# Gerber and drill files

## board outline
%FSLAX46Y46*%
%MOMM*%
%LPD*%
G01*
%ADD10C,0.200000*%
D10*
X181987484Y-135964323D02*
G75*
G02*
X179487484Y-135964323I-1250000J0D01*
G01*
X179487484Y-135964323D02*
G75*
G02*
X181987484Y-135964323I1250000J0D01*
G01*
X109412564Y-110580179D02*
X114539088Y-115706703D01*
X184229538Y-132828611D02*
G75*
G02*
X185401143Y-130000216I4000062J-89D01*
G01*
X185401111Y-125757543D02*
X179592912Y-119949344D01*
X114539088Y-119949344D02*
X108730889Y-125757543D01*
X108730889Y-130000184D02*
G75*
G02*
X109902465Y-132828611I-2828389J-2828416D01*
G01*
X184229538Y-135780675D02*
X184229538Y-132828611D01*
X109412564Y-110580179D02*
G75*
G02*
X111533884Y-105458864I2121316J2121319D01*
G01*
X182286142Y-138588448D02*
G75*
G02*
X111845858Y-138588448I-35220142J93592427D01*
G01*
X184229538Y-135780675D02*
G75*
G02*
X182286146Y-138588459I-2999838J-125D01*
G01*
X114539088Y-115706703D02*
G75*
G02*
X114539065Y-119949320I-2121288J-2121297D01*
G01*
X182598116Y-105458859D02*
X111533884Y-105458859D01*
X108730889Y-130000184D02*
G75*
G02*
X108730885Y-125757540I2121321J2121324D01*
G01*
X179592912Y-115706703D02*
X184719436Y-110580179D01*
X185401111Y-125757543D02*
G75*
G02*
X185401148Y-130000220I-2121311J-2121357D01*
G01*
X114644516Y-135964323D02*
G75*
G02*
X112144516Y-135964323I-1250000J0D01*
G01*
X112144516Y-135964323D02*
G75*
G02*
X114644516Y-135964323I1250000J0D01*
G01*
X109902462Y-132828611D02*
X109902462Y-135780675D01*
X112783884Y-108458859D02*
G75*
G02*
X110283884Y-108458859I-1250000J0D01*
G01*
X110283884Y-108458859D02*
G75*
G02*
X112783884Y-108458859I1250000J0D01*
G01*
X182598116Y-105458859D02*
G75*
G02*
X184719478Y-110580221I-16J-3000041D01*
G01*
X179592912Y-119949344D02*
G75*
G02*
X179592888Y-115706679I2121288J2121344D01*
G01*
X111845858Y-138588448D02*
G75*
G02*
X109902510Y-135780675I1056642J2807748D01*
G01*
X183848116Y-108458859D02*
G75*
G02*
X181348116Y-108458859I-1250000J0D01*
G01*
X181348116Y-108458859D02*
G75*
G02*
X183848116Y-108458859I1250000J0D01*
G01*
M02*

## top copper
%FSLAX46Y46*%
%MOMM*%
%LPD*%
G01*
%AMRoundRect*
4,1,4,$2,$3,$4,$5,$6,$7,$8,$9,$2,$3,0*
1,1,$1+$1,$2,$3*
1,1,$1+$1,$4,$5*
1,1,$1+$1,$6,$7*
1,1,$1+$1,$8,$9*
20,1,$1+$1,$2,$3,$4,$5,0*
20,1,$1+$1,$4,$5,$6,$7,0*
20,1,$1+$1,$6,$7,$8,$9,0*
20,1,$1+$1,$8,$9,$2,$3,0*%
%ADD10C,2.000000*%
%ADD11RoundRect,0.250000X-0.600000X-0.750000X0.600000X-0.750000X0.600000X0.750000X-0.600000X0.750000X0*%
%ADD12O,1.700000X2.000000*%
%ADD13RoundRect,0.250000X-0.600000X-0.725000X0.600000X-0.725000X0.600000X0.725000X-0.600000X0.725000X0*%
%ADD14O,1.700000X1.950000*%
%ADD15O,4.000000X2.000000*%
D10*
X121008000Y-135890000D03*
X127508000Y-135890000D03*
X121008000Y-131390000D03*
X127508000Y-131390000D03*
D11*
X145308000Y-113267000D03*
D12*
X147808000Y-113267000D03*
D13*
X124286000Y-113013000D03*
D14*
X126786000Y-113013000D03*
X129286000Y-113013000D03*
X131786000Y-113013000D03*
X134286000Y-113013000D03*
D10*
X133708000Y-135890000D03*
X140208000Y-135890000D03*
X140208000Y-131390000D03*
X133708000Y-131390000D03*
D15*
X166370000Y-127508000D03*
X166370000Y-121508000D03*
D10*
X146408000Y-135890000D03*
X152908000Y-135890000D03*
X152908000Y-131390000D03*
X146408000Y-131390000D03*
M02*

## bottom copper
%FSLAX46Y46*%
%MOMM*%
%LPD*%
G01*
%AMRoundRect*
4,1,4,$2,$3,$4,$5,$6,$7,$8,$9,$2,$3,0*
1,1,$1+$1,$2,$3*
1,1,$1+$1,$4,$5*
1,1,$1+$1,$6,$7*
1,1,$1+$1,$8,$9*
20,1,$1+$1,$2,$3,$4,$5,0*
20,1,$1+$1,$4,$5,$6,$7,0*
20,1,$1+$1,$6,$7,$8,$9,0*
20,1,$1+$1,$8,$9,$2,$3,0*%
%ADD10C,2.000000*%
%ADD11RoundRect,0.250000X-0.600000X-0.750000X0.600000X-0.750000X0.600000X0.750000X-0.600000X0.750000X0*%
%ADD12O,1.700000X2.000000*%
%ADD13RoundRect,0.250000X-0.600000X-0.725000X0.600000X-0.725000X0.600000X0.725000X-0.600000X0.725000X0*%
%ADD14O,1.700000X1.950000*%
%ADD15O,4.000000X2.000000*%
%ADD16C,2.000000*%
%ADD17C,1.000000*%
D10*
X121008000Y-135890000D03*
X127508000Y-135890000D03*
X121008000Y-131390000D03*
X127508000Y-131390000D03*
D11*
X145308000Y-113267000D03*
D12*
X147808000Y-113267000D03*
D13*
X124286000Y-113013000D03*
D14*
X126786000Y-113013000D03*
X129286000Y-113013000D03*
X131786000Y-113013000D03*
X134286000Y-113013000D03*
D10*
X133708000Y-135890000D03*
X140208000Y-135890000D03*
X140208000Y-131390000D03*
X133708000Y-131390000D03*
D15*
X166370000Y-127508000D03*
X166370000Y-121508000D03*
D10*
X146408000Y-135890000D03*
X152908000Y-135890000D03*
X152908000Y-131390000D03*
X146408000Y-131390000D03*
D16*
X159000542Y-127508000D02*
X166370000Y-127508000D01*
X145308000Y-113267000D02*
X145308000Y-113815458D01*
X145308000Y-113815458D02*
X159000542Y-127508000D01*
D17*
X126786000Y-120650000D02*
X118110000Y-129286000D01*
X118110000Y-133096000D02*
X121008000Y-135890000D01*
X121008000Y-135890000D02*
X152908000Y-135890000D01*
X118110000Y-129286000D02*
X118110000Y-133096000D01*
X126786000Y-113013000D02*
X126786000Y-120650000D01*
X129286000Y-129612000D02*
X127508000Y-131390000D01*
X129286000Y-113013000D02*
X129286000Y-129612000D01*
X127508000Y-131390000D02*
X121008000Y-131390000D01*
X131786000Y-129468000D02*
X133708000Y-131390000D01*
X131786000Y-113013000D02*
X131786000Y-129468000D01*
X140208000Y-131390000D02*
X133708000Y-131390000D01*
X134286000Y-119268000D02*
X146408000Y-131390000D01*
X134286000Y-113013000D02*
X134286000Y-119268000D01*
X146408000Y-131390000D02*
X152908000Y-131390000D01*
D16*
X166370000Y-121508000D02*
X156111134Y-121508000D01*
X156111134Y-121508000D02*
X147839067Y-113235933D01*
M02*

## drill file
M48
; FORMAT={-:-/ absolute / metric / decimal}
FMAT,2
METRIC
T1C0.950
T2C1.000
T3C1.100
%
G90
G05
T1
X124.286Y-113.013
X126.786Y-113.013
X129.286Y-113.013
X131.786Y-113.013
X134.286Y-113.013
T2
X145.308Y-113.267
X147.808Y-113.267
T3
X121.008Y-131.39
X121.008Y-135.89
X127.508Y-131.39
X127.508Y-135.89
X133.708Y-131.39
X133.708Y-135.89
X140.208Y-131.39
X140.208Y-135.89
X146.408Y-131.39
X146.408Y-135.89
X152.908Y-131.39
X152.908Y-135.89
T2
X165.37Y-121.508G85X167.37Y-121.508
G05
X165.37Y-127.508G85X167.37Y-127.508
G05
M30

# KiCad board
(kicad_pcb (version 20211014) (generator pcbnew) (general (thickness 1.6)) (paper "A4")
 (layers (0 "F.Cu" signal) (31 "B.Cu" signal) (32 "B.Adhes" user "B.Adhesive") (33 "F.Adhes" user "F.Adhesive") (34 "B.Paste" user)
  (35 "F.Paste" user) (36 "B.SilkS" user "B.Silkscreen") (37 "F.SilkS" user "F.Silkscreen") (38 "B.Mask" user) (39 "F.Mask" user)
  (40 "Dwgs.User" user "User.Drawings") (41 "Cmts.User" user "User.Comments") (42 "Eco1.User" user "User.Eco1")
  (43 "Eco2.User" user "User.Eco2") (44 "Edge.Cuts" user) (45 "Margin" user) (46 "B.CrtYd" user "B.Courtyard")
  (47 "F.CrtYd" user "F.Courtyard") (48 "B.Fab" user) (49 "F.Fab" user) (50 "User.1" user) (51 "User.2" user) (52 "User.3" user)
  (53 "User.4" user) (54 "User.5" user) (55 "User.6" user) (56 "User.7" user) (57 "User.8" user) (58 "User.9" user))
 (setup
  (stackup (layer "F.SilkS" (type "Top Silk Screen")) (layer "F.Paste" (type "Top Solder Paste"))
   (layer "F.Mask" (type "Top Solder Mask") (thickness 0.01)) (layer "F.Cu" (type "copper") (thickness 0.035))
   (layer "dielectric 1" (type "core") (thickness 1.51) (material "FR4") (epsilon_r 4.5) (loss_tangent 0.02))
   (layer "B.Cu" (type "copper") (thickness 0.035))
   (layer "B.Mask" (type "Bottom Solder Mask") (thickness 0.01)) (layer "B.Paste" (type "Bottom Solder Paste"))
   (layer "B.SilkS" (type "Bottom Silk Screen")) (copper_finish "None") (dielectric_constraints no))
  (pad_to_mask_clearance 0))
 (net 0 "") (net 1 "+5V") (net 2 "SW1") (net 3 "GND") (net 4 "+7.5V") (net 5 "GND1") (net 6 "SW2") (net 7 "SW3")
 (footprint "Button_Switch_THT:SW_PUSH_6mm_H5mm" (layer "F.Cu") (at 127.508 135.89 180)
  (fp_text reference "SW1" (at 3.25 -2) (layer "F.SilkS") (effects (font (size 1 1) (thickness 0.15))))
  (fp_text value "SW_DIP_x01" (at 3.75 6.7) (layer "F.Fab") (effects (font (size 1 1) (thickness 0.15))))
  (pad "1" thru_hole circle (at 6.5 0 270) (size 2 2) (drill 1.1) (layers *.Cu *.Mask) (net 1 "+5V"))
  (pad "1" thru_hole circle (at 0 0 270) (size 2 2) (drill 1.1) (layers *.Cu *.Mask) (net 1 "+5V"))
  (pad "2" thru_hole circle (at 6.5 4.5 270) (size 2 2) (drill 1.1) (layers *.Cu *.Mask) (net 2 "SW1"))
  (pad "2" thru_hole circle (at 0 4.5 270) (size 2 2) (drill 1.1) (layers *.Cu *.Mask) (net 2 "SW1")))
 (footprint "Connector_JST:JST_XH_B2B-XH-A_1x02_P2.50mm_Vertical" (layer "F.Cu") (at 145.308 113.267)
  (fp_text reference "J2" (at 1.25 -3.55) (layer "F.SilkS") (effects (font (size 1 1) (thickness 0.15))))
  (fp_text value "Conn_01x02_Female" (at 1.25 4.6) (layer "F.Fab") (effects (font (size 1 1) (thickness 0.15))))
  (pad "1" thru_hole roundrect (at 0 0) (size 1.7 2) (drill 1) (layers *.Cu *.Mask) (roundrect_rratio 0.1470588235) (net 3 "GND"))
  (pad "2" thru_hole oval (at 2.5 0) (size 1.7 2) (drill 1) (layers *.Cu *.Mask) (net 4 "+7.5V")))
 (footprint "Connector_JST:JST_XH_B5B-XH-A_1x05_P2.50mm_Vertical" (layer "F.Cu") (at 124.286 113.013)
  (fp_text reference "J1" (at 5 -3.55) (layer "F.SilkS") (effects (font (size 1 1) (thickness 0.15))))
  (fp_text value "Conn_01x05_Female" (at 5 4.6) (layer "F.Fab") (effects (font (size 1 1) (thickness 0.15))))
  (pad "1" thru_hole roundrect (at 0 0) (size 1.7 1.95) (drill 0.95) (layers *.Cu *.Mask) (roundrect_rratio 0.1470588235) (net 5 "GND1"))
  (pad "2" thru_hole oval (at 2.5 0) (size 1.7 1.95) (drill 0.95) (layers *.Cu *.Mask) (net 1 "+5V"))
  (pad "3" thru_hole oval (at 5 0) (size 1.7 1.95) (drill 0.95) (layers *.Cu *.Mask) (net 2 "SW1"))
  (pad "4" thru_hole oval (at 7.5 0) (size 1.7 1.95) (drill 0.95) (layers *.Cu *.Mask) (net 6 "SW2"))
  (pad "5" thru_hole oval (at 10 0) (size 1.7 1.95) (drill 0.95) (layers *.Cu *.Mask) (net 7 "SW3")))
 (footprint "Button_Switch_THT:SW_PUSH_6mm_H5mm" (layer "F.Cu") (at 140.208 135.89 180)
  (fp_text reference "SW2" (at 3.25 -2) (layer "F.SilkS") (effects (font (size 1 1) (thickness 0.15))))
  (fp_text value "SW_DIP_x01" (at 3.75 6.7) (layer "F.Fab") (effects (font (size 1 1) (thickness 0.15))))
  (pad "1" thru_hole circle (at 6.5 0 270) (size 2 2) (drill 1.1) (layers *.Cu *.Mask) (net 1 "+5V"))
  (pad "1" thru_hole circle (at 0 0 270) (size 2 2) (drill 1.1) (layers *.Cu *.Mask) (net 1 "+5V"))
  (pad "2" thru_hole circle (at 0 4.5 270) (size 2 2) (drill 1.1) (layers *.Cu *.Mask) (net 6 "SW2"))
  (pad "2" thru_hole circle (at 6.5 4.5 270) (size 2 2) (drill 1.1) (layers *.Cu *.Mask) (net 6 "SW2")))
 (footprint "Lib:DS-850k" (layer "F.Cu") (at 166.37 127.508 -90)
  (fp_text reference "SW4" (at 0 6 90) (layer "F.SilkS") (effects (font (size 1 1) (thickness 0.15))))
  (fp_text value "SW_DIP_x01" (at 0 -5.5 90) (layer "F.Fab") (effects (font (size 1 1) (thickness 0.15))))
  (pad "1" thru_hole oval locked (at 0 0) (size 4 2) (drill oval 3 1) (layers *.Cu *.Mask) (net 3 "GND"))
  (pad "2" thru_hole oval locked (at -6 0) (size 4 2) (drill oval 3 1) (layers *.Cu *.Mask) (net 4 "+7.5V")))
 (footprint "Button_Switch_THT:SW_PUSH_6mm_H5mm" (layer "F.Cu") (at 152.908 135.89 180)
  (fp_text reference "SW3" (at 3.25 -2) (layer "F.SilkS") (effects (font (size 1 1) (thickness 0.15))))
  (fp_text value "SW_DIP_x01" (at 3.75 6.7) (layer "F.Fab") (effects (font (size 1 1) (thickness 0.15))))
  (pad "1" thru_hole circle (at 6.5 0 270) (size 2 2) (drill 1.1) (layers *.Cu *.Mask) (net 1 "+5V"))
  (pad "1" thru_hole circle (at 0 0 270) (size 2 2) (drill 1.1) (layers *.Cu *.Mask) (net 1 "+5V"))
  (pad "2" thru_hole circle (at 0 4.5 270) (size 2 2) (drill 1.1) (layers *.Cu *.Mask) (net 7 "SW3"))
  (pad "2" thru_hole circle (at 6.5 4.5 270) (size 2 2) (drill 1.1) (layers *.Cu *.Mask) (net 7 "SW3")))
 (gr_circle (center 180.737484 135.964323) (end 181.987484 135.964323) (layer "Edge.Cuts") (width 0.2) (fill none))
 (gr_line (start 109.412564 110.580179) (end 114.539088 115.706703) (layer "Edge.Cuts") (width 0.2))
 (gr_arc (start 184.229538 132.828611) (mid 184.534027 131.297882) (end 185.401111 130.000184) (layer "Edge.Cuts") (width 0.2))
 (gr_line (start 185.401111 125.757543) (end 179.592912 119.949344) (layer "Edge.Cuts") (width 0.2))
 (gr_line (start 114.539088 119.949344) (end 108.730889 125.757543) (layer "Edge.Cuts") (width 0.2))
 (gr_arc (start 108.730889 130.000184) (mid 109.59798 131.297877) (end 109.902462 132.828611) (layer "Edge.Cuts") (width 0.2))
 (gr_line (start 184.229538 135.780675) (end 184.229538 132.828611) (layer "Edge.Cuts") (width 0.2))
 (gr_arc (start 109.412564 110.580179) (mid 108.762246 107.310809) (end 111.533884 105.458859) (layer "Edge.Cuts") (width 0.2))
 (gr_arc (start 182.286142 138.588448) (mid 147.066 144.996025) (end 111.845858 138.588448) (layer "Edge.Cuts") (width 0.2))
 (gr_arc (start 184.229538 135.780675) (mid 183.696321 137.488069) (end 182.286142 138.588448) (layer "Edge.Cuts") (width 0.2))
 (gr_arc (start 114.539088 115.706703) (mid 115.417768 117.828024) (end 114.539088 119.949344) (layer "Edge.Cuts") (width 0.2))
 (gr_line (start 182.598116 105.458859) (end 111.533884 105.458859) (layer "Edge.Cuts") (width 0.2))
 (gr_arc (start 108.730889 130.000184) (mid 107.852209 127.878864) (end 108.730889 125.757543) (layer "Edge.Cuts") (width 0.2))
 (gr_line (start 179.592912 115.706703) (end 184.719436 110.580179) (layer "Edge.Cuts") (width 0.2))
 (gr_arc (start 185.401111 125.757543) (mid 186.279792 127.878864) (end 185.401111 130.000184) (layer "Edge.Cuts") (width 0.2))
 (gr_circle (center 113.394516 135.964323) (end 114.644516 135.964323) (layer "Edge.Cuts") (width 0.2) (fill none))
 (gr_line (start 109.902462 132.828611) (end 109.902462 135.780675) (layer "Edge.Cuts") (width 0.2))
 (gr_circle (center 111.533884 108.458859) (end 112.783884 108.458859) (layer "Edge.Cuts") (width 0.2) (fill none))
 (gr_arc (start 182.598116 105.458859) (mid 185.369755 107.310807) (end 184.719436 110.580179) (layer "Edge.Cuts") (width 0.2))
 (gr_arc (start 179.592912 119.949344) (mid 178.714233 117.828024) (end 179.592912 115.706703) (layer "Edge.Cuts") (width 0.2))
 (gr_arc (start 111.845858 138.588448) (mid 110.435702 137.48804) (end 109.902462 135.780675) (layer "Edge.Cuts") (width 0.2))
 (gr_circle (center 182.598116 108.458859) (end 183.848116 108.458859) (layer "Edge.Cuts") (width 0.2) (fill none))
 (segment (start 159.000542 127.508) (end 166.37 127.508) (width 2) (layer "B.Cu") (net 3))
 (segment (start 145.308 113.267) (end 145.308 113.815458) (width 2) (layer "B.Cu") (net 3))
 (segment (start 145.308 113.815458) (end 159.000542 127.508) (width 2) (layer "B.Cu") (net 3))
 (segment (start 126.786 120.65) (end 118.11 129.286) (width 1) (layer "B.Cu") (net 1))
 (segment (start 118.11 133.096) (end 121.008 135.89) (width 1) (layer "B.Cu") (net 1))
 (segment (start 121.008 135.89) (end 152.908 135.89) (width 1) (layer "B.Cu") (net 1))
 (segment (start 118.11 129.286) (end 118.11 133.096) (width 1) (layer "B.Cu") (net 1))
 (segment (start 126.786 113.013) (end 126.786 120.65) (width 1) (layer "B.Cu") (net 1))
 (segment (start 129.286 129.612) (end 127.508 131.39) (width 1) (layer "B.Cu") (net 2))
 (segment (start 129.286 113.013) (end 129.286 129.612) (width 1) (layer "B.Cu") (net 2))
 (segment (start 127.508 131.39) (end 121.008 131.39) (width 1) (layer "B.Cu") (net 2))
 (segment (start 131.786 129.468) (end 133.708 131.39) (width 1) (layer "B.Cu") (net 6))
 (segment (start 131.786 113.013) (end 131.786 129.468) (width 1) (layer "B.Cu") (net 6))
 (segment (start 140.208 131.39) (end 133.708 131.39) (width 1) (layer "B.Cu") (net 6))
 (segment (start 134.286 119.268) (end 146.408 131.39) (width 1) (layer "B.Cu") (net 7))
 (segment (start 134.286 113.013) (end 134.286 119.268) (width 1) (layer "B.Cu") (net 7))
 (segment (start 146.408 131.39) (end 152.908 131.39) (width 1) (layer "B.Cu") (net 7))
 (segment (start 166.37 121.508) (end 156.111134 121.508) (width 2) (layer "B.Cu") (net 4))
 (segment (start 156.111134 121.508) (end 147.839067 113.235933) (width 2) (layer "B.Cu") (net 4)))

